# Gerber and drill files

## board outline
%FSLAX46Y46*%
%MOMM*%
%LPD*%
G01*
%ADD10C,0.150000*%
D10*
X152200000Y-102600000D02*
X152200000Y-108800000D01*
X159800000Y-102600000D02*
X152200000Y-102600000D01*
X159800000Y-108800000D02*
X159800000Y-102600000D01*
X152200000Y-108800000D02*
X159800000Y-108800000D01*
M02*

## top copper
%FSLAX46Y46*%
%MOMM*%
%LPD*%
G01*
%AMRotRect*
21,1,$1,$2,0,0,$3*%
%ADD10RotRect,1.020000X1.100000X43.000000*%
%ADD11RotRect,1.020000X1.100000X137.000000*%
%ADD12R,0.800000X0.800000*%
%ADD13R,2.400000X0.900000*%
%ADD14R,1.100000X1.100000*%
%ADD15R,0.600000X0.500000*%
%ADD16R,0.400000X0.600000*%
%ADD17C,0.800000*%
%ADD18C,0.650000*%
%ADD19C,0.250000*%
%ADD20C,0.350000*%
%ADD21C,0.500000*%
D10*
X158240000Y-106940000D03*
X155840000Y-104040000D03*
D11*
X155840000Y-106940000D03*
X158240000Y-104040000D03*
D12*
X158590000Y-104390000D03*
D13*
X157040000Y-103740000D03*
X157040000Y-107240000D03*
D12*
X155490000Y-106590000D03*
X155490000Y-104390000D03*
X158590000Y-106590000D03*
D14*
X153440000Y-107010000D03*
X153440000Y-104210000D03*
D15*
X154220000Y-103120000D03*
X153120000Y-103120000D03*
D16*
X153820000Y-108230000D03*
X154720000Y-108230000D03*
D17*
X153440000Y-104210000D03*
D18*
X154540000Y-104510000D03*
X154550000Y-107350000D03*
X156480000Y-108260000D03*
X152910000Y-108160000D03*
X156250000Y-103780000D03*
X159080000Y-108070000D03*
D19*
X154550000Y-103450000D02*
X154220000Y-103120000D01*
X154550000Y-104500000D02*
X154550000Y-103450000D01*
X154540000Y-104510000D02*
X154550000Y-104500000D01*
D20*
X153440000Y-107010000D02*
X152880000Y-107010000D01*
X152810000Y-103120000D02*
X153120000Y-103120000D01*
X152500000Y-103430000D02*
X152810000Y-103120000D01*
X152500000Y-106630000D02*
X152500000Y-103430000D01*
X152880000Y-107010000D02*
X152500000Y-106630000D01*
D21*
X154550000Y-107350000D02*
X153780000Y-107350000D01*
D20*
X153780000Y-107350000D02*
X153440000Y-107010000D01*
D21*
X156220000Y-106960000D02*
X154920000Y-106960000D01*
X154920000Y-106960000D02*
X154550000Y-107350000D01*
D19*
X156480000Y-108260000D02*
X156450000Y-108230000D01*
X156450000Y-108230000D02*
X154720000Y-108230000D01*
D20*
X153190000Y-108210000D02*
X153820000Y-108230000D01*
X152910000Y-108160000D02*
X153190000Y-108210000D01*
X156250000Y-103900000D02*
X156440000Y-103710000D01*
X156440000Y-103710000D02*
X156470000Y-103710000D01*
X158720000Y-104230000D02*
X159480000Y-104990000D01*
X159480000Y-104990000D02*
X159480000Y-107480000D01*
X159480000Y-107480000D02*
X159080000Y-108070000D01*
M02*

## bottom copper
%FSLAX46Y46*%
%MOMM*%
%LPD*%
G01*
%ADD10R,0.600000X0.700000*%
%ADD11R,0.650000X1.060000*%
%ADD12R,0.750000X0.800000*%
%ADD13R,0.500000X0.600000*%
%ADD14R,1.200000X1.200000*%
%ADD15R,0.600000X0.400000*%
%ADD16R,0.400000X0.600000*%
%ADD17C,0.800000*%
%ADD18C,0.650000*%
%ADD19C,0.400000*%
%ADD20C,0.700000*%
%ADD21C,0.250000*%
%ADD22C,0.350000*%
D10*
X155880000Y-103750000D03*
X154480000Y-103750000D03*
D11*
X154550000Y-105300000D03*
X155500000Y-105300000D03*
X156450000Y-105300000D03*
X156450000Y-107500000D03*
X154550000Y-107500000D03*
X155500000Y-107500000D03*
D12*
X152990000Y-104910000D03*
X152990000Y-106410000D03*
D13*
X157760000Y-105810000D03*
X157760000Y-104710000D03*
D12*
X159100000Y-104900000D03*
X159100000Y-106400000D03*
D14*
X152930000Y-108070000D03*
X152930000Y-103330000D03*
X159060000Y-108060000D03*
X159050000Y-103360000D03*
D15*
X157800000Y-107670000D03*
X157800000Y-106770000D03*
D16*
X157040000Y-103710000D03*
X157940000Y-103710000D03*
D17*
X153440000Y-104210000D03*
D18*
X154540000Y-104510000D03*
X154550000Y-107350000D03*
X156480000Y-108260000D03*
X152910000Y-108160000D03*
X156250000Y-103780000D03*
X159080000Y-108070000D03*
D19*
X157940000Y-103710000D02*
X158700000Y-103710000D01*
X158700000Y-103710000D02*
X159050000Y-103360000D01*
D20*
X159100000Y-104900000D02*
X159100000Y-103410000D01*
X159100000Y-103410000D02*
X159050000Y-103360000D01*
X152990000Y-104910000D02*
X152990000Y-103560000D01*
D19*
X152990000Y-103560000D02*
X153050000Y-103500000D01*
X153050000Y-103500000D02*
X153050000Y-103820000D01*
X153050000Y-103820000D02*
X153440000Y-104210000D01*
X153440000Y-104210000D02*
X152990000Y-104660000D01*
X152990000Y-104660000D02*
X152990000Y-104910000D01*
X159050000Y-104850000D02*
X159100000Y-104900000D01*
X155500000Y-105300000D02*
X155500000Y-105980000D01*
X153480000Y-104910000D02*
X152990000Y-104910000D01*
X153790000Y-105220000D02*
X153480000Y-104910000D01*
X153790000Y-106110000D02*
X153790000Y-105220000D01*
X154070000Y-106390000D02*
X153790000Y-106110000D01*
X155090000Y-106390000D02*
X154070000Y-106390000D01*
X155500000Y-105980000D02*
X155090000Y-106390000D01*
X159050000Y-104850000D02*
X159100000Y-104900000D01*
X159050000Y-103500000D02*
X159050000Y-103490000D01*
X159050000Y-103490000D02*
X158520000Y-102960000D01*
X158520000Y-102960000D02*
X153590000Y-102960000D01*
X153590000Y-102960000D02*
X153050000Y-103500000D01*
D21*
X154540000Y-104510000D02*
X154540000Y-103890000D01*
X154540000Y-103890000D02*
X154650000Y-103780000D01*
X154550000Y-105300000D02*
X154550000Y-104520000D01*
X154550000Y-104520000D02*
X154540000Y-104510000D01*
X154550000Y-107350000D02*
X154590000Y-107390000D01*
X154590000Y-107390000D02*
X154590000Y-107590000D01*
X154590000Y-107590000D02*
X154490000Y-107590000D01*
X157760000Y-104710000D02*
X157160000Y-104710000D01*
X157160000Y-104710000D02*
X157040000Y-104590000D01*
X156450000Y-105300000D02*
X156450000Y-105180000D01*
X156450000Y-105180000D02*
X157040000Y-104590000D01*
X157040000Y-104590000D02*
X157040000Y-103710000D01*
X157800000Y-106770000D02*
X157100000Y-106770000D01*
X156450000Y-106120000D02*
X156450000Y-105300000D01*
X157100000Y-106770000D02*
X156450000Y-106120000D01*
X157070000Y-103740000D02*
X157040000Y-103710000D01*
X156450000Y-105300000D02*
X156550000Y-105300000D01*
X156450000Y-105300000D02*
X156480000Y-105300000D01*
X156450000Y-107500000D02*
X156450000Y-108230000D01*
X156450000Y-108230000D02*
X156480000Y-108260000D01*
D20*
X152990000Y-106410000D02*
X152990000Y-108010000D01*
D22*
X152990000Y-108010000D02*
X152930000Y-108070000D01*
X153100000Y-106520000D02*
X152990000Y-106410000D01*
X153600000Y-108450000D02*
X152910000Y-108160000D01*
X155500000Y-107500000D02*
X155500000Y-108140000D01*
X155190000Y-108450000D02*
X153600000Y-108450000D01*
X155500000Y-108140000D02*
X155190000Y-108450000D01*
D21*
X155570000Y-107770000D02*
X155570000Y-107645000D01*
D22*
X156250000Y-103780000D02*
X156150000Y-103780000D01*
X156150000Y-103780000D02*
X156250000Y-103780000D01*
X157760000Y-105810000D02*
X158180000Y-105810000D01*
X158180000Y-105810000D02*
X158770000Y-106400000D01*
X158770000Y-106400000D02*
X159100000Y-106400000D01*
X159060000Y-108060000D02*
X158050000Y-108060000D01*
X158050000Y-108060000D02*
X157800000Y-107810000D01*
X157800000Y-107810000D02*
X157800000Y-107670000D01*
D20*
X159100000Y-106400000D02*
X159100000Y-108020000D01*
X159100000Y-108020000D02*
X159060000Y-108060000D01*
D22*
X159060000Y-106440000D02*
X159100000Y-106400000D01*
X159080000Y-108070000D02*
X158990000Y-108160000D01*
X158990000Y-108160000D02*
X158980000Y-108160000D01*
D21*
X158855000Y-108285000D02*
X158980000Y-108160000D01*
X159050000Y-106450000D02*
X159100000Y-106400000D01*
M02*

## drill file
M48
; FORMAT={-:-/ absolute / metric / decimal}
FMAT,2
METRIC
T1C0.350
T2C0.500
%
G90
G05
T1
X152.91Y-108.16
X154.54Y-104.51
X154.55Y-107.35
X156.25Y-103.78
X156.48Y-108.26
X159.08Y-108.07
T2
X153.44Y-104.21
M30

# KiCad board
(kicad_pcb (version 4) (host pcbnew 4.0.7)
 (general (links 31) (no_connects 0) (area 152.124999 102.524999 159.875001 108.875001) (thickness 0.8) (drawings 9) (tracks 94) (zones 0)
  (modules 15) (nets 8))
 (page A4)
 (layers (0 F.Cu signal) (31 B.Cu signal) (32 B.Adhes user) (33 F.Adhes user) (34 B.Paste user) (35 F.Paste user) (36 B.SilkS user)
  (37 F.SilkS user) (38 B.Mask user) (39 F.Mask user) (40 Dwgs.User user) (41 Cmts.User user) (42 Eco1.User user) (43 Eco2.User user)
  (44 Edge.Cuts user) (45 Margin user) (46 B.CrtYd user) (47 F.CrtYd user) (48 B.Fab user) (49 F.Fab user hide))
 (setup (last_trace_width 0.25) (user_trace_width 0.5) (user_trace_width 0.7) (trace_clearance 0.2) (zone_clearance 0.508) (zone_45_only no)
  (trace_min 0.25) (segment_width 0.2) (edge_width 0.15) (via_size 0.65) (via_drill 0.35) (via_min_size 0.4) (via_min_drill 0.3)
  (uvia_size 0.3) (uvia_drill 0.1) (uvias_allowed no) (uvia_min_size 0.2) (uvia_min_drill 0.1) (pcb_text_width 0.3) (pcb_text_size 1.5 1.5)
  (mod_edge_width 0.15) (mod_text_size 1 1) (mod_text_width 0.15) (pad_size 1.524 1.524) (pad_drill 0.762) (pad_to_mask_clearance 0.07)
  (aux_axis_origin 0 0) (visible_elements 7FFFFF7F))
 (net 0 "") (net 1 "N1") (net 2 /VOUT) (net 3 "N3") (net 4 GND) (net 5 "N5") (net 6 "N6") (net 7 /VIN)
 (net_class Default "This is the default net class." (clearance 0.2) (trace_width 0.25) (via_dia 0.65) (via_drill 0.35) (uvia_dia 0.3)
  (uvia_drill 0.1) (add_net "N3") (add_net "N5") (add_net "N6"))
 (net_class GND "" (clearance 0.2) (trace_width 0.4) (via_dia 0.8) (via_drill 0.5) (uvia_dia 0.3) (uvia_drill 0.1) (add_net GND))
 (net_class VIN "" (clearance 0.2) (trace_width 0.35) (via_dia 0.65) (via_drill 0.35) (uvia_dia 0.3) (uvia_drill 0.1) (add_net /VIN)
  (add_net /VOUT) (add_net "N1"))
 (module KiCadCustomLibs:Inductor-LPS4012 (layer F.Cu) (at 157.04 105.49 90)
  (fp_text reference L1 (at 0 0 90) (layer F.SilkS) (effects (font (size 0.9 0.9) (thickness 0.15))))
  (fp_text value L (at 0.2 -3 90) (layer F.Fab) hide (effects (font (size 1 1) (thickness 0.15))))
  (pad 1 smd rect (at -1.45 1.2 43) (size 1.02 1.1) (layers F.Cu F.Paste F.Mask) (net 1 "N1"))
  (pad 2 smd rect (at 1.45 -1.2 43) (size 1.02 1.1) (layers F.Cu F.Paste F.Mask) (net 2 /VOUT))
  (pad 1 smd rect (at -1.45 -1.2 137) (size 1.02 1.1) (layers F.Cu F.Paste F.Mask) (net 1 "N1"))
  (pad 2 smd rect (at 1.45 1.2 137) (size 1.02 1.1) (layers F.Cu F.Paste F.Mask) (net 2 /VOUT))
  (pad 2 smd rect (at 1.1 1.55 90) (size 0.8 0.8) (layers F.Cu F.Paste F.Mask) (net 2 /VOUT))
  (pad 2 smd rect (at 1.75 0 90) (size 0.9 2.4) (layers F.Cu F.Paste F.Mask) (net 2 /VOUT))
  (pad 1 smd rect (at -1.75 0 90) (size 0.9 2.4) (layers F.Cu F.Paste F.Mask) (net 1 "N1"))
  (pad 1 smd rect (at -1.1 -1.55 90) (size 0.8 0.8) (layers F.Cu F.Paste F.Mask) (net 1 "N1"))
  (pad 2 smd rect (at 1.1 -1.55 90) (size 0.8 0.8) (layers F.Cu F.Paste F.Mask) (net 2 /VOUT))
  (pad 1 smd rect (at -1.1 1.55 90) (size 0.8 0.8) (layers F.Cu F.Paste F.Mask) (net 1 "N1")))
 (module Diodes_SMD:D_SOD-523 (layer B.Cu) (at 155.18 103.75)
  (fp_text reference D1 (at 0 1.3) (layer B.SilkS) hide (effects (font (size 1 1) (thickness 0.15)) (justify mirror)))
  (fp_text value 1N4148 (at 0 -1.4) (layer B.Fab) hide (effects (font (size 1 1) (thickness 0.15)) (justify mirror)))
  (pad 2 smd rect (at 0.7 0 180) (size 0.6 0.7) (layers B.Cu B.Paste B.Mask) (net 2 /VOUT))
  (pad 1 smd rect (at -0.7 0 180) (size 0.6 0.7) (layers B.Cu B.Paste B.Mask) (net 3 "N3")))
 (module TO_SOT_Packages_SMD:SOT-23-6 (layer B.Cu) (at 155.5 106.4 270)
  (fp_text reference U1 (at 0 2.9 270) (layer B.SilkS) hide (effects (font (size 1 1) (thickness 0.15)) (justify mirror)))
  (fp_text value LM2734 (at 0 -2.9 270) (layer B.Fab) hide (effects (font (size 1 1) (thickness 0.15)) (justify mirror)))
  (pad 1 smd rect (at -1.1 0.95 270) (size 1.06 0.65) (layers B.Cu B.Paste B.Mask) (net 3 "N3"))
  (pad 2 smd rect (at -1.1 0 270) (size 1.06 0.65) (layers B.Cu B.Paste B.Mask) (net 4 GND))
  (pad 3 smd rect (at -1.1 -0.95 270) (size 1.06 0.65) (layers B.Cu B.Paste B.Mask) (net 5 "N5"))
  (pad 4 smd rect (at 1.1 -0.95 270) (size 1.06 0.65) (layers B.Cu B.Paste B.Mask) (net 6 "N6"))
  (pad 6 smd rect (at 1.1 0.95 270) (size 1.06 0.65) (layers B.Cu B.Paste B.Mask) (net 1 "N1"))
  (pad 5 smd rect (at 1.1 0 270) (size 1.06 0.65) (layers B.Cu B.Paste B.Mask) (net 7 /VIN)))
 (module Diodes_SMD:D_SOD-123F (layer F.Cu) (at 153.44 105.61 90)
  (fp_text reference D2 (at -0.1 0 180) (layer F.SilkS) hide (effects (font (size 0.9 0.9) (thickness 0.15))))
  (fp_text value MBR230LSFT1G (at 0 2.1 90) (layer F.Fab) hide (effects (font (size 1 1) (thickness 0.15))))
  (pad 1 smd rect (at -1.4 0 90) (size 1.1 1.1) (layers F.Cu F.Paste F.Mask) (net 1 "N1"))
  (pad 2 smd rect (at 1.4 0 90) (size 1.1 1.1) (layers F.Cu F.Paste F.Mask) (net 4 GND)))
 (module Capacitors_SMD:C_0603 (layer B.Cu) (at 152.99 105.66 90)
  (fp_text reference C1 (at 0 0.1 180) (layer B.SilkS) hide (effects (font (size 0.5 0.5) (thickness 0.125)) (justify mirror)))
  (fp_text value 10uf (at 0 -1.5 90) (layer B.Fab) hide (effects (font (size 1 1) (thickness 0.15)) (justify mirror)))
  (pad 2 smd rect (at 0.75 0 90) (size 0.8 0.75) (layers B.Cu B.Paste B.Mask) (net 4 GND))
  (pad 1 smd rect (at -0.75 0 90) (size 0.8 0.75) (layers B.Cu B.Paste B.Mask) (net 7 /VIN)))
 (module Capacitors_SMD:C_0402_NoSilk (layer F.Cu) (at 153.67 103.12 180)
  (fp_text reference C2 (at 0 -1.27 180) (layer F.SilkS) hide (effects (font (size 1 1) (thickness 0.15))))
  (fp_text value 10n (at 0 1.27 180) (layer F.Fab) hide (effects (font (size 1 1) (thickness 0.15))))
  (pad 1 smd rect (at -0.55 0 180) (size 0.6 0.5) (layers F.Cu F.Paste F.Mask) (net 3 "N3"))
  (pad 2 smd rect (at 0.55 0 180) (size 0.6 0.5) (layers F.Cu F.Paste F.Mask) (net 1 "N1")))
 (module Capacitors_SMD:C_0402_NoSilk (layer B.Cu) (at 157.76 105.26 90)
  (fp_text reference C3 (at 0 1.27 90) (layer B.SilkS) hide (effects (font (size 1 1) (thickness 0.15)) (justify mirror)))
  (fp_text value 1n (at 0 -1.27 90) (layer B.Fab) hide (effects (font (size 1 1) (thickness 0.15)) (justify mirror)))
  (pad 1 smd rect (at -0.55 0 90) (size 0.6 0.5) (layers B.Cu B.Paste B.Mask) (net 2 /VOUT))
  (pad 2 smd rect (at 0.55 0 90) (size 0.6 0.5) (layers B.Cu B.Paste B.Mask) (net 5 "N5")))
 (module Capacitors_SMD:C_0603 (layer B.Cu) (at 159.1 105.65 90)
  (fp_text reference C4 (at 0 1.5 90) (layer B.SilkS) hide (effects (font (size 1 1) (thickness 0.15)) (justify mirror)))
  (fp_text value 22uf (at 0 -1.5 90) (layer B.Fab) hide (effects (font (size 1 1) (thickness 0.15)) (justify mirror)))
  (pad 2 smd rect (at 0.75 0 90) (size 0.8 0.75) (layers B.Cu B.Paste B.Mask) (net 4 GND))
  (pad 1 smd rect (at -0.75 0 90) (size 0.8 0.75) (layers B.Cu B.Paste B.Mask) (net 2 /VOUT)))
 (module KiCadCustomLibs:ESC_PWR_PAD (layer B.Cu) (at 152.93 108.07)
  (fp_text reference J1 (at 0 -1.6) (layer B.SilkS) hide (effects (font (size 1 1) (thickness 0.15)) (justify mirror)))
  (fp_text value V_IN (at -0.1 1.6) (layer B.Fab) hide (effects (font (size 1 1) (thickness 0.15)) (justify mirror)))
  (pad 1 smd rect (at 0 0) (size 1.2 1.2) (layers B.Cu B.Paste B.Mask) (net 7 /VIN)))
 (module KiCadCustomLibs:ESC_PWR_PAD (layer B.Cu) (at 152.93 103.33)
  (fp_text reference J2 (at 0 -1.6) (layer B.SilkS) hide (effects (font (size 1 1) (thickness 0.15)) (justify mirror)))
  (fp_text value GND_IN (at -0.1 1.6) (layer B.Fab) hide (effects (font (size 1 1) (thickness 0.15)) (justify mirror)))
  (pad 1 smd rect (at 0 0) (size 1.2 1.2) (layers B.Cu B.Paste B.Mask) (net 4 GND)))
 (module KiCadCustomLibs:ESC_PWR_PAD (layer B.Cu) (at 159.06 108.06)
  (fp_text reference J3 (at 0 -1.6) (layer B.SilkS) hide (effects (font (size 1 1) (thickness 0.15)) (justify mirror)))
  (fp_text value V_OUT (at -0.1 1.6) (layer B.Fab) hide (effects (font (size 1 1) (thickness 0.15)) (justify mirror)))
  (pad 1 smd rect (at 0 0) (size 1.2 1.2) (layers B.Cu B.Paste B.Mask) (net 2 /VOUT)))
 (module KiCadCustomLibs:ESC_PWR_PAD (layer B.Cu) (at 159.05 103.36)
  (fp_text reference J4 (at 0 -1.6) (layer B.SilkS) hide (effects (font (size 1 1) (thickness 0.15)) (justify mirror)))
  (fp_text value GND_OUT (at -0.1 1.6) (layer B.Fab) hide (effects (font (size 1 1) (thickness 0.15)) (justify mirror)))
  (pad 1 smd rect (at 0 0) (size 1.2 1.2) (layers B.Cu B.Paste B.Mask) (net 4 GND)))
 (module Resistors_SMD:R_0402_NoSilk (layer F.Cu) (at 154.27 108.23)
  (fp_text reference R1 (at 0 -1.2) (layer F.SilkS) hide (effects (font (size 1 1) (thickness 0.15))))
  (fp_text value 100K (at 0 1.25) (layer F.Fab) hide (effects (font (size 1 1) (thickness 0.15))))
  (pad 1 smd rect (at -0.45 0) (size 0.4 0.6) (layers F.Cu F.Paste F.Mask) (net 7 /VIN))
  (pad 2 smd rect (at 0.45 0) (size 0.4 0.6) (layers F.Cu F.Paste F.Mask) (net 6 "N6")))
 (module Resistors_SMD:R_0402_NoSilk (layer B.Cu) (at 157.8 107.22 90)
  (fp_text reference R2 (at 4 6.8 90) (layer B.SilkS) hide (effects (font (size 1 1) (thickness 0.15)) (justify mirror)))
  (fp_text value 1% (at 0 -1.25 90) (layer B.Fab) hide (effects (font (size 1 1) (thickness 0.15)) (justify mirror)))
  (pad 1 smd rect (at -0.45 0 90) (size 0.4 0.6) (layers B.Cu B.Paste B.Mask) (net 2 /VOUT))
  (pad 2 smd rect (at 0.45 0 90) (size 0.4 0.6) (layers B.Cu B.Paste B.Mask) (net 5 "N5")))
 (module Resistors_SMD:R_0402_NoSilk (layer B.Cu) (at 157.49 103.71)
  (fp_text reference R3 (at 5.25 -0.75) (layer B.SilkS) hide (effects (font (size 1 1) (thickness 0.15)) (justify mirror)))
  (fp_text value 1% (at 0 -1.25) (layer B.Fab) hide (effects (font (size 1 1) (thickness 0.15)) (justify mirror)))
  (pad 1 smd rect (at -0.45 0) (size 0.4 0.6) (layers B.Cu B.Paste B.Mask) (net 5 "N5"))
  (pad 2 smd rect (at 0.45 0) (size 0.4 0.6) (layers B.Cu B.Paste B.Mask) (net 4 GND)))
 (gr_line (start 152.2 102.6) (end 152.2 108.8) (angle 90) (layer Edge.Cuts) (width 0.15))
 (gr_line (start 159.8 102.6) (end 152.2 102.6) (angle 90) (layer Edge.Cuts) (width 0.15))
 (gr_line (start 159.8 108.8) (end 159.8 102.6) (angle 90) (layer Edge.Cuts) (width 0.15))
 (gr_line (start 152.2 108.8) (end 159.8 108.8) (angle 90) (layer Edge.Cuts) (width 0.15))
 (segment (start 157.94 103.71) (end 158.7 103.71) (width 0.4) (layer B.Cu) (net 4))
 (segment (start 158.7 103.71) (end 159.05 103.36) (width 0.4) (layer B.Cu) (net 4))
 (segment (start 159.1 104.9) (end 159.1 103.41) (width 0.7) (layer B.Cu) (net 4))
 (segment (start 159.1 103.41) (end 159.05 103.36) (width 0.7) (layer B.Cu) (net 4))
 (segment (start 152.99 104.91) (end 152.99 103.56) (width 0.7) (layer B.Cu) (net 4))
 (segment (start 152.99 103.56) (end 153.05 103.5) (width 0.4) (layer B.Cu) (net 4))
 (segment (start 153.05 103.5) (end 153.05 103.82) (width 0.4) (layer B.Cu) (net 4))
 (segment (start 153.05 103.82) (end 153.44 104.21) (width 0.4) (layer B.Cu) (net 4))
 (segment (start 153.44 104.21) (end 152.99 104.66) (width 0.4) (layer B.Cu) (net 4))
 (via (at 153.44 104.21) (size 0.8) (drill 0.5) (layers F.Cu B.Cu) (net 4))
 (segment (start 152.99 104.66) (end 152.99 104.91) (width 0.4) (layer B.Cu) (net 4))
 (segment (start 159.05 104.85) (end 159.1 104.9) (width 0.4) (layer B.Cu) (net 4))
 (segment (start 155.5 105.3) (end 155.5 105.98) (width 0.4) (layer B.Cu) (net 4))
 (segment (start 153.48 104.91) (end 152.99 104.91) (width 0.4) (layer B.Cu) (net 4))
 (segment (start 153.79 105.22) (end 153.48 104.91) (width 0.4) (layer B.Cu) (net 4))
 (segment (start 153.79 106.11) (end 153.79 105.22) (width 0.4) (layer B.Cu) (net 4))
 (segment (start 154.07 106.39) (end 153.79 106.11) (width 0.4) (layer B.Cu) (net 4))
 (segment (start 155.09 106.39) (end 154.07 106.39) (width 0.4) (layer B.Cu) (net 4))
 (segment (start 155.5 105.98) (end 155.09 106.39) (width 0.4) (layer B.Cu) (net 4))
 (segment (start 159.05 104.85) (end 159.1 104.9) (width 0.4) (layer B.Cu) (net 4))
 (segment (start 159.05 103.5) (end 159.05 103.49) (width 0.4) (layer B.Cu) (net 4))
 (segment (start 159.05 103.49) (end 158.52 102.96) (width 0.4) (layer B.Cu) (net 4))
 (segment (start 158.52 102.96) (end 153.59 102.96) (width 0.4) (layer B.Cu) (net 4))
 (segment (start 153.59 102.96) (end 153.05 103.5) (width 0.4) (layer B.Cu) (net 4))
 (segment (start 154.54 104.51) (end 154.54 103.89) (width 0.25) (layer B.Cu) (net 3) (status 20))
 (segment (start 154.54 103.89) (end 154.65 103.78) (width 0.25) (layer B.Cu) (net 3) (status 30))
 (segment (start 154.55 105.3) (end 154.55 104.52) (width 0.25) (layer B.Cu) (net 3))
 (segment (start 154.55 103.45) (end 154.22 103.12) (width 0.25) (layer F.Cu) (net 3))
 (segment (start 154.55 104.5) (end 154.55 103.45) (width 0.25) (layer F.Cu) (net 3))
 (segment (start 154.54 104.51) (end 154.55 104.5) (width 0.25) (layer F.Cu) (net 3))
 (via (at 154.54 104.51) (size 0.65) (drill 0.35) (layers F.Cu B.Cu) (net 3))
 (segment (start 154.55 104.52) (end 154.54 104.51) (width 0.25) (layer B.Cu) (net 3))
 (segment (start 153.44 107.01) (end 152.88 107.01) (width 0.35) (layer F.Cu) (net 1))
 (segment (start 152.81 103.12) (end 153.12 103.12) (width 0.35) (layer F.Cu) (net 1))
 (segment (start 152.5 103.43) (end 152.81 103.12) (width 0.35) (layer F.Cu) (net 1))
 (segment (start 152.5 106.63) (end 152.5 103.43) (width 0.35) (layer F.Cu) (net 1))
 (segment (start 152.88 107.01) (end 152.5 106.63) (width 0.35) (layer F.Cu) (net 1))
 (segment (start 154.55 107.35) (end 153.78 107.35) (width 0.5) (layer F.Cu) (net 1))
 (segment (start 153.78 107.35) (end 153.44 107.01) (width 0.35) (layer F.Cu) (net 1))
 (segment (start 156.22 106.96) (end 154.92 106.96) (width 0.5) (layer F.Cu) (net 1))
 (segment (start 154.55 107.35) (end 154.59 107.39) (width 0.25) (layer B.Cu) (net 1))
 (via (at 154.55 107.35) (size 0.65) (drill 0.35) (layers F.Cu B.Cu) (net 1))
 (segment (start 154.92 106.96) (end 154.55 107.35) (width 0.5) (layer F.Cu) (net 1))
 (segment (start 154.59 107.39) (end 154.59 107.59) (width 0.25) (layer B.Cu) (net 1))
 (segment (start 154.59 107.59) (end 154.49 107.59) (width 0.25) (layer B.Cu) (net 1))
 (segment (start 157.76 104.71) (end 157.16 104.71) (width 0.25) (layer B.Cu) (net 5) (status 10))
 (segment (start 157.16 104.71) (end 157.04 104.59) (width 0.25) (layer B.Cu) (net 5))
 (segment (start 156.45 105.3) (end 156.45 105.18) (width 0.25) (layer B.Cu) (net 5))
 (segment (start 156.45 105.18) (end 157.04 104.59) (width 0.25) (layer B.Cu) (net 5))
 (segment (start 157.04 104.59) (end 157.04 103.71) (width 0.25) (layer B.Cu) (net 5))
 (segment (start 157.8 106.77) (end 157.1 106.77) (width 0.25) (layer B.Cu) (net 5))
 (segment (start 156.45 106.12) (end 156.45 105.3) (width 0.25) (layer B.Cu) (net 5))
 (segment (start 157.1 106.77) (end 156.45 106.12) (width 0.25) (layer B.Cu) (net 5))
 (segment (start 157.07 103.74) (end 157.04 103.71) (width 0.25) (layer B.Cu) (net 5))
 (segment (start 156.45 105.3) (end 156.55 105.3) (width 0.25) (layer B.Cu) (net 5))
 (segment (start 156.45 105.3) (end 156.48 105.3) (width 0.25) (layer B.Cu) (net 5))
 (segment (start 156.45 107.5) (end 156.45 108.23) (width 0.25) (layer B.Cu) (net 6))
 (segment (start 156.45 108.23) (end 156.48 108.26) (width 0.25) (layer B.Cu) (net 6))
 (via (at 156.48 108.26) (size 0.65) (drill 0.35) (layers F.Cu B.Cu) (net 6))
 (segment (start 156.48 108.26) (end 156.45 108.23) (width 0.25) (layer F.Cu) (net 6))
 (segment (start 156.45 108.23) (end 154.72 108.23) (width 0.25) (layer F.Cu) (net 6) (status 20))
 (segment (start 152.99 106.41) (end 152.99 108.01) (width 0.7) (layer B.Cu) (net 7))
 (segment (start 152.99 108.01) (end 152.93 108.07) (width 0.35) (layer B.Cu) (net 7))
 (segment (start 153.1 106.52) (end 152.99 106.41) (width 0.35) (layer B.Cu) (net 7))
 (via (at 152.91 108.16) (size 0.65) (drill 0.35) (layers F.Cu B.Cu) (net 7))
 (segment (start 153.6 108.45) (end 152.91 108.16) (width 0.35) (layer B.Cu) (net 7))
 (segment (start 153.19 108.21) (end 153.82 108.23) (width 0.35) (layer F.Cu) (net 7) (status 20))
 (segment (start 152.91 108.16) (end 153.19 108.21) (width 0.35) (layer F.Cu) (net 7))
 (segment (start 155.5 107.5) (end 155.5 108.14) (width 0.35) (layer B.Cu) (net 7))
 (segment (start 155.19 108.45) (end 153.6 108.45) (width 0.35) (layer B.Cu) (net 7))
 (segment (start 155.5 108.14) (end 155.19 108.45) (width 0.35) (layer B.Cu) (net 7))
 (segment (start 155.57 107.77) (end 155.57 107.645) (width 0.25) (layer B.Cu) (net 7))
 (segment (start 156.25 103.78) (end 156.15 103.78) (width 0.35) (layer B.Cu) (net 2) (status 30))
 (segment (start 156.15 103.78) (end 156.25 103.78) (width 0.35) (layer B.Cu) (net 2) (status 30))
 (via (at 156.25 103.78) (size 0.65) (drill 0.35) (layers F.Cu B.Cu) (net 2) (status 30))
 (segment (start 156.25 103.9) (end 156.44 103.71) (width 0.35) (layer F.Cu) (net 2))
 (segment (start 156.44 103.71) (end 156.47 103.71) (width 0.35) (layer F.Cu) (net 2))
 (segment (start 157.76 105.81) (end 158.18 105.81) (width 0.35) (layer B.Cu) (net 2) (status 10))
 (segment (start 158.18 105.81) (end 158.77 106.4) (width 0.35) (layer B.Cu) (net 2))
 (segment (start 158.77 106.4) (end 159.1 106.4) (width 0.35) (layer B.Cu) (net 2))
 (segment (start 159.06 108.06) (end 158.05 108.06) (width 0.35) (layer B.Cu) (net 2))
 (segment (start 158.05 108.06) (end 157.8 107.81) (width 0.35) (layer B.Cu) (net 2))
 (segment (start 157.8 107.81) (end 157.8 107.67) (width 0.35) (layer B.Cu) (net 2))
 (segment (start 159.1 106.4) (end 159.1 108.02) (width 0.7) (layer B.Cu) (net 2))
 (segment (start 159.1 108.02) (end 159.06 108.06) (width 0.7) (layer B.Cu) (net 2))
 (segment (start 159.06 106.44) (end 159.1 106.4) (width 0.35) (layer B.Cu) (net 2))
 (segment (start 158.72 104.23) (end 159.48 104.99) (width 0.35) (layer F.Cu) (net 2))
 (segment (start 159.48 104.99) (end 159.48 107.48) (width 0.35) (layer F.Cu) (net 2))
 (segment (start 159.48 107.48) (end 159.08 108.07) (width 0.35) (layer F.Cu) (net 2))
 (via (at 159.08 108.07) (size 0.65) (drill 0.35) (layers F.Cu B.Cu) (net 2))
 (segment (start 159.08 108.07) (end 158.99 108.16) (width 0.35) (layer B.Cu) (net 2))
 (segment (start 158.99 108.16) (end 158.98 108.16) (width 0.35) (layer B.Cu) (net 2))
 (segment (start 158.855 108.285) (end 158.98 108.16) (width 0.25) (layer B.Cu) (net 2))
 (segment (start 159.05 106.45) (end 159.1 106.4) (width 0.25) (layer B.Cu) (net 2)))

